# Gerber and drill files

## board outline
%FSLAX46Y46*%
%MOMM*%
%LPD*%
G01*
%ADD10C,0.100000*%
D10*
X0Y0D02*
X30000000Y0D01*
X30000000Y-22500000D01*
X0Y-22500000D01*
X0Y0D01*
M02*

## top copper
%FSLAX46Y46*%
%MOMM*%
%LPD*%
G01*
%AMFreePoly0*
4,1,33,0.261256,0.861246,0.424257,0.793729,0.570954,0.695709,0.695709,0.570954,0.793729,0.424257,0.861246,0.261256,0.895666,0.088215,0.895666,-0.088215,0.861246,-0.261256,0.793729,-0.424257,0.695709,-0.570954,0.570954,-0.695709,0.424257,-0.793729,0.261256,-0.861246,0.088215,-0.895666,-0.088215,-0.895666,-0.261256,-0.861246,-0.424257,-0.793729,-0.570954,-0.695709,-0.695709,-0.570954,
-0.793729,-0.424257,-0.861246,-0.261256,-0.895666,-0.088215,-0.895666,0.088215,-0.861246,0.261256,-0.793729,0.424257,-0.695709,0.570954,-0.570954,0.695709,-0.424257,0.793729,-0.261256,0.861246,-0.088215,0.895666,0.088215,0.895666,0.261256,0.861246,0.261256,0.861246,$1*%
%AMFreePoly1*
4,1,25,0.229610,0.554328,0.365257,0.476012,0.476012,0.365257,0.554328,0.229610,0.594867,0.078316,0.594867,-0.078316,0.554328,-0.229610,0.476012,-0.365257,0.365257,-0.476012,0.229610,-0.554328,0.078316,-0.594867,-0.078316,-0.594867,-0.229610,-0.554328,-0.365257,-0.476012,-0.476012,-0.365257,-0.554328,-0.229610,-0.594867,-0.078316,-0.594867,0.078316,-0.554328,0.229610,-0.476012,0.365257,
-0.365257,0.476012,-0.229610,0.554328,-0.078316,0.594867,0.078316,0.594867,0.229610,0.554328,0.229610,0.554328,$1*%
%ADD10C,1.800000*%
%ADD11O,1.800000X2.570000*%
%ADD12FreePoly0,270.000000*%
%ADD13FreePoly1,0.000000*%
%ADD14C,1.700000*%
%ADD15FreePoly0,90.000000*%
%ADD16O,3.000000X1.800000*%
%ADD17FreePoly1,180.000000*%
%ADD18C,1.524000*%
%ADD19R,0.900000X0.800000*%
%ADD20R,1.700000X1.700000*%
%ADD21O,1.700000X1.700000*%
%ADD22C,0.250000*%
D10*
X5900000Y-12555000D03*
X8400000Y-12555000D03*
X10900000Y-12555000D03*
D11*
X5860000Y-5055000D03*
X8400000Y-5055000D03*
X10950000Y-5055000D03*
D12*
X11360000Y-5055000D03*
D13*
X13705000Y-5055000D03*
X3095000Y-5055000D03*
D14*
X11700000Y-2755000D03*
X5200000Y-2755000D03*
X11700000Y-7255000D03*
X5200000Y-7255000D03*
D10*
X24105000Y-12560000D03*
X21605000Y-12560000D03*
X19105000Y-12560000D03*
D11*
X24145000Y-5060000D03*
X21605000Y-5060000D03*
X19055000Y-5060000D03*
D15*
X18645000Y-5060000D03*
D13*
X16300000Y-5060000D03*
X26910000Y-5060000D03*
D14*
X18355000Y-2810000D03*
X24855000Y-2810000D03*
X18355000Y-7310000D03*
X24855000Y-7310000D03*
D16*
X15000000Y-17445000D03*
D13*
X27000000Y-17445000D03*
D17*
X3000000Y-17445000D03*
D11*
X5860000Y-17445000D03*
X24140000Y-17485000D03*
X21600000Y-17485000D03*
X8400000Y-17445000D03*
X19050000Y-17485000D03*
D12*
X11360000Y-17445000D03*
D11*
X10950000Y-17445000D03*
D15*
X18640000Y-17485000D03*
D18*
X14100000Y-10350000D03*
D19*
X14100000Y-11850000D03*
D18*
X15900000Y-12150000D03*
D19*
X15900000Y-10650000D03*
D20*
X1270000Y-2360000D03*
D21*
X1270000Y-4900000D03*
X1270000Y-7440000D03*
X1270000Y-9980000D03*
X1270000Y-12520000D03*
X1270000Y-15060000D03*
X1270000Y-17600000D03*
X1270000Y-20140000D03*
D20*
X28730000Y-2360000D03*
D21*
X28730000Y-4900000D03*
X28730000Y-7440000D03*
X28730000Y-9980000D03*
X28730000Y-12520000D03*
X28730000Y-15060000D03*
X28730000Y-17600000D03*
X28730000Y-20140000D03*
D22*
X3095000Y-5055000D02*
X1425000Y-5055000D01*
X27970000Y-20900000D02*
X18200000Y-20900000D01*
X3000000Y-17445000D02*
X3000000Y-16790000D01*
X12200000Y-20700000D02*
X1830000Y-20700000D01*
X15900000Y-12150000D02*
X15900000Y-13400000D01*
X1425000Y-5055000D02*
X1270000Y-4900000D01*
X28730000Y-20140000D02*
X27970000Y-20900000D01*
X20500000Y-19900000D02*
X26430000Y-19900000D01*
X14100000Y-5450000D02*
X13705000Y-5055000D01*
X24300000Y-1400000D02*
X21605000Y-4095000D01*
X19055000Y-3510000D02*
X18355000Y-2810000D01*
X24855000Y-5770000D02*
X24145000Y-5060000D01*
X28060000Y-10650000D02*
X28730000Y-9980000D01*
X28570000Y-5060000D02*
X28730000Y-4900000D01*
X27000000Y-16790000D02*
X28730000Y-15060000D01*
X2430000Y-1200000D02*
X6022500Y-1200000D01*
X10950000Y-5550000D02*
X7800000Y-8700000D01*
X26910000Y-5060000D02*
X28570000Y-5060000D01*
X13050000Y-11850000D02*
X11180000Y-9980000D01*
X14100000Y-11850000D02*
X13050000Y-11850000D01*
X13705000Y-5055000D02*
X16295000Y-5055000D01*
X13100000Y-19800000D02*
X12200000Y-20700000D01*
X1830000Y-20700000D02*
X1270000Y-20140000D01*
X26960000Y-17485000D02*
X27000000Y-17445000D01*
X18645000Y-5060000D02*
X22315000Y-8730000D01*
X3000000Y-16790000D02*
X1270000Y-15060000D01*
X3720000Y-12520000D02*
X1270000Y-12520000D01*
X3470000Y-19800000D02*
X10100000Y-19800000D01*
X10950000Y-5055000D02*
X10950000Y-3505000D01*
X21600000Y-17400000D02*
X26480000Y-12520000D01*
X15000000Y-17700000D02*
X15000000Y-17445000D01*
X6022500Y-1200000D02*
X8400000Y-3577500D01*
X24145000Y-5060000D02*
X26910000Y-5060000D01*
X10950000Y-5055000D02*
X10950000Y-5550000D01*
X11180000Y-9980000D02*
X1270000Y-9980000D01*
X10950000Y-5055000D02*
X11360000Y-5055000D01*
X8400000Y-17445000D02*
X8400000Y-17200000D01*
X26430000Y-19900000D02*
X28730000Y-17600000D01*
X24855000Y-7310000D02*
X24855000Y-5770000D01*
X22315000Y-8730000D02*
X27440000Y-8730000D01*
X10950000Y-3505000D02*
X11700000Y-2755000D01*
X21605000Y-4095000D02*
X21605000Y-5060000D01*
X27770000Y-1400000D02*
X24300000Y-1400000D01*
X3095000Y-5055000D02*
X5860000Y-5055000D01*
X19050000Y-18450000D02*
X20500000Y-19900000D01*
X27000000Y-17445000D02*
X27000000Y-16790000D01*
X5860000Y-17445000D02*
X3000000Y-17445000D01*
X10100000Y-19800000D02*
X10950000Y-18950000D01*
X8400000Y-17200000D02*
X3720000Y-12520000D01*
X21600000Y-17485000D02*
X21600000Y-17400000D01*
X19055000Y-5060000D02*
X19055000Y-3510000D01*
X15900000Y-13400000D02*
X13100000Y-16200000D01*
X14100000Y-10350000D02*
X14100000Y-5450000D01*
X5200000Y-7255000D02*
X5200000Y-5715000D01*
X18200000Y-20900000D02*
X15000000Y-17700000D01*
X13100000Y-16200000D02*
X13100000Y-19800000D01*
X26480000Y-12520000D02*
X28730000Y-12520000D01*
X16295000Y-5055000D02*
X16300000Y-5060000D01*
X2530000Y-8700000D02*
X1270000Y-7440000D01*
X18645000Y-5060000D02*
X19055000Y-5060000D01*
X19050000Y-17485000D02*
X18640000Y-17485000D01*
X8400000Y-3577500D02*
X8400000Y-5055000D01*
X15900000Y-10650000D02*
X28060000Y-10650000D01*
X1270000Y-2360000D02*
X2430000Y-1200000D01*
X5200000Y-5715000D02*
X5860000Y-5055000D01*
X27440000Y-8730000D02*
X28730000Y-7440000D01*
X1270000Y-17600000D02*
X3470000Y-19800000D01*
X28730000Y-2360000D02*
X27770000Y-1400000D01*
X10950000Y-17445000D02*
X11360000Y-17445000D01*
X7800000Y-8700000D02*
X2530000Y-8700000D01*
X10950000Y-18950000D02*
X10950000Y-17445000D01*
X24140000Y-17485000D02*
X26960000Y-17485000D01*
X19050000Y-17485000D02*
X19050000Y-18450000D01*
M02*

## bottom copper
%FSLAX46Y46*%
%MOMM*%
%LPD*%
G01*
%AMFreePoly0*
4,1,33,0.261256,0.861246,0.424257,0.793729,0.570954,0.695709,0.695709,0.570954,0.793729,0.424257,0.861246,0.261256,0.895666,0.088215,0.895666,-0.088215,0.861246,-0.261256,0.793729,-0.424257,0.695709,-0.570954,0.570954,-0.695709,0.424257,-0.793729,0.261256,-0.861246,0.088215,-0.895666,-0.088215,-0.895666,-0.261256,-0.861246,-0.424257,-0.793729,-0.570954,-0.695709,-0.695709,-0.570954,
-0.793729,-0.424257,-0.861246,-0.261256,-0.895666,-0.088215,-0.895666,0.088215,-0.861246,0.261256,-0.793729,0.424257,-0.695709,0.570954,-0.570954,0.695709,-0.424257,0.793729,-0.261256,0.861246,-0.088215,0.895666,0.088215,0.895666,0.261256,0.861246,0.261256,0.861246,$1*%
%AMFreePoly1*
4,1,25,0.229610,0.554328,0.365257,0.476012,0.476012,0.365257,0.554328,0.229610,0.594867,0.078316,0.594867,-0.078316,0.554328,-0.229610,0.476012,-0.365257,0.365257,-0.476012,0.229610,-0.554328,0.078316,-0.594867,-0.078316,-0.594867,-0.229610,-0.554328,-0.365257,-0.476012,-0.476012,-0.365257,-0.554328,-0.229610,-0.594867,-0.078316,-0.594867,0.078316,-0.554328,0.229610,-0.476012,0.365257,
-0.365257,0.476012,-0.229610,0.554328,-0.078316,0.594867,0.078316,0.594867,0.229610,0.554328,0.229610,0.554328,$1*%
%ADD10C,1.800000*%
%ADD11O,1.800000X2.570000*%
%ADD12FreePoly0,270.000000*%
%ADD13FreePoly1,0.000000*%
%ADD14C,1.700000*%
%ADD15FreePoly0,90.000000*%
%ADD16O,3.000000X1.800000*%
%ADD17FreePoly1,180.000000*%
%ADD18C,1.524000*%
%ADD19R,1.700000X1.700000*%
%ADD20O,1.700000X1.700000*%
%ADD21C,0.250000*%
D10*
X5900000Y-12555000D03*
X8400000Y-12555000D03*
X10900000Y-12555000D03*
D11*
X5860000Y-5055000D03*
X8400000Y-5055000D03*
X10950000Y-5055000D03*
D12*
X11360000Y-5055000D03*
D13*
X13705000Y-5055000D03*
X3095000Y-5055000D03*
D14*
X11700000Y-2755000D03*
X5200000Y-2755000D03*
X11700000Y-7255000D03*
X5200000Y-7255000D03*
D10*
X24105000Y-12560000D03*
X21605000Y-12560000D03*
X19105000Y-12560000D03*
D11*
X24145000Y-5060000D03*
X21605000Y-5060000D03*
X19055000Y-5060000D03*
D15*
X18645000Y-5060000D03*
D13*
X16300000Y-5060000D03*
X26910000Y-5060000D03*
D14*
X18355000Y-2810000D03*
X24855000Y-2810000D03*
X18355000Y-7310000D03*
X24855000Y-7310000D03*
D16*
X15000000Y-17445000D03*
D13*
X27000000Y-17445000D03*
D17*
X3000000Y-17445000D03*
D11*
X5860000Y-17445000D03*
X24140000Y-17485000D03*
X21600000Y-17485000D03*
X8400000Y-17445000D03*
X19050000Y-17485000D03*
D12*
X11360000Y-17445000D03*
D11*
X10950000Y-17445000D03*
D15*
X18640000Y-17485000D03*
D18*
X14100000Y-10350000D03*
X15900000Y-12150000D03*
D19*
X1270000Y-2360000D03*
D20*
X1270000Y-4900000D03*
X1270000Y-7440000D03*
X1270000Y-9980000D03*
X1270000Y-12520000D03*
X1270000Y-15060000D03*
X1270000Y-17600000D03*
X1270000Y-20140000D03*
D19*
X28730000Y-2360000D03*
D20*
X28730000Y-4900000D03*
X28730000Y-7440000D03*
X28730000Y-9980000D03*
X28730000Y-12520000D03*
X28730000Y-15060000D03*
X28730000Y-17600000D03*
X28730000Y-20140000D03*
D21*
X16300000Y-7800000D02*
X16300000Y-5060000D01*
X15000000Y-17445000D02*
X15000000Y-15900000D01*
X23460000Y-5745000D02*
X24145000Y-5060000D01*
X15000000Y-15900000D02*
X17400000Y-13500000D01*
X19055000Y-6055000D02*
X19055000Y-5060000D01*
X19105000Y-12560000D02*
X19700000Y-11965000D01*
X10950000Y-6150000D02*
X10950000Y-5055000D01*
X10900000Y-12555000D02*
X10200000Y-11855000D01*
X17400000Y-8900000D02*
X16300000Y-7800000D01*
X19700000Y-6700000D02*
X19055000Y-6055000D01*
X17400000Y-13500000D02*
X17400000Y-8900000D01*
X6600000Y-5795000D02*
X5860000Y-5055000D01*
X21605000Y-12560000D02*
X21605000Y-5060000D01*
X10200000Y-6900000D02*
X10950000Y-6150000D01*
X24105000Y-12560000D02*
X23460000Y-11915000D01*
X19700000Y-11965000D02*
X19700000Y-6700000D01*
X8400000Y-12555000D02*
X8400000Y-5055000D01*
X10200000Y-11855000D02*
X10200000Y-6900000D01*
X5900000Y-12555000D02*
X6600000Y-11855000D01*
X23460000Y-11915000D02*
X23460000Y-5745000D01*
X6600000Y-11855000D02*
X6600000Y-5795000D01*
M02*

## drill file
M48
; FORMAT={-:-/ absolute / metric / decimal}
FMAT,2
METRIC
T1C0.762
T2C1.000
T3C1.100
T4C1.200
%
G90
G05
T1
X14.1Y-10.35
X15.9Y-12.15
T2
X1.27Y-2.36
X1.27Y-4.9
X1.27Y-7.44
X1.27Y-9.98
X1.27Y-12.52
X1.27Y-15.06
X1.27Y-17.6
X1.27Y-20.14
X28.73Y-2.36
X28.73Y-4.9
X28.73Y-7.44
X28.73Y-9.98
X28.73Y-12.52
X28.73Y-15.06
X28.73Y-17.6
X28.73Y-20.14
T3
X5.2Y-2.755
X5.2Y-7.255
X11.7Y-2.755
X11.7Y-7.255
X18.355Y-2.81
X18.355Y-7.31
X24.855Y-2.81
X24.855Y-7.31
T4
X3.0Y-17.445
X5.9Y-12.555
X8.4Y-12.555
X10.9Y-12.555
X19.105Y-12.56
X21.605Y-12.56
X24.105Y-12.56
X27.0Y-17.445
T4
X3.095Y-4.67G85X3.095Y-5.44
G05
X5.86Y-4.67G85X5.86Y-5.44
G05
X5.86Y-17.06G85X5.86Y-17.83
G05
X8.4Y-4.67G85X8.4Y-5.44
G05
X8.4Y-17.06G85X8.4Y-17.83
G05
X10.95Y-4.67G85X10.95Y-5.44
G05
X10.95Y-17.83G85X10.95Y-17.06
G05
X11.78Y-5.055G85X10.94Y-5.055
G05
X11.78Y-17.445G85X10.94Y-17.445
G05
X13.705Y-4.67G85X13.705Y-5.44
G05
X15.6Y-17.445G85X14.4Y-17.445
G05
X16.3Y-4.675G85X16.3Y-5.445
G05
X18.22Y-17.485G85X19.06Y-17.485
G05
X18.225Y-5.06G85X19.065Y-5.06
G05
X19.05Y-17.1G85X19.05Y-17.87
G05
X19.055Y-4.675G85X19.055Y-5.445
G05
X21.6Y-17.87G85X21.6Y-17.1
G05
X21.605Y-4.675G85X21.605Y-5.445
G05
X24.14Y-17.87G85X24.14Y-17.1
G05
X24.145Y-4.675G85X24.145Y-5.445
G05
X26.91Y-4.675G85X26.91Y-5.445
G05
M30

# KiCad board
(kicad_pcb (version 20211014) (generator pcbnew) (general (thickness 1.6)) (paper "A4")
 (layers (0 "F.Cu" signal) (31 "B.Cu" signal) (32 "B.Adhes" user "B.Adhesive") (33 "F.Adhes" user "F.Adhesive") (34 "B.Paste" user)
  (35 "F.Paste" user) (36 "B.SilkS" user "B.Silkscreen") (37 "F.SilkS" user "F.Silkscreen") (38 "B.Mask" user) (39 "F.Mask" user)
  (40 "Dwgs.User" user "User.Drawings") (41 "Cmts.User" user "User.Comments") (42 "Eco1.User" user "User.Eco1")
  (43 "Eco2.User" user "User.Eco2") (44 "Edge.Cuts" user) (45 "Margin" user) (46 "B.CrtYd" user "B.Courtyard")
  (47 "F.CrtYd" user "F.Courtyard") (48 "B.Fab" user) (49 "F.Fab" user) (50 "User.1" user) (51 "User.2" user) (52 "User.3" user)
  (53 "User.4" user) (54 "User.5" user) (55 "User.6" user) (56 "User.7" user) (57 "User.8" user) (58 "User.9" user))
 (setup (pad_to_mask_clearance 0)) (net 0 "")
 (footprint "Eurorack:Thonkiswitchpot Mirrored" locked (layer "F.Cu") (at 8.4 5.055)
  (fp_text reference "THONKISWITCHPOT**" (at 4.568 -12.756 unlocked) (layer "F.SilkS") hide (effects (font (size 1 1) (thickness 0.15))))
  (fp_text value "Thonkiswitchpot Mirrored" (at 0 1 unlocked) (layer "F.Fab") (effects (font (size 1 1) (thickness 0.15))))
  (pad "1" thru_hole circle locked (at -2.5 7.5 270) (size 1.8 1.8) (drill 1.2) (layers *.Cu *.Mask))
  (pad "2" thru_hole circle locked (at 0 7.5 270) (size 1.8 1.8) (drill 1.2) (layers *.Cu *.Mask))
  (pad "3" thru_hole circle locked (at 2.5 7.5 270) (size 1.8 1.8) (drill 1.2) (layers *.Cu *.Mask))
  (pad "4" thru_hole oval locked (at -2.54 0) (size 1.8 2.57) (drill oval 1.2 1.97) (layers *.Cu *.Mask))
  (pad "5" thru_hole oval locked (at 0 0) (size 1.8 2.57) (drill oval 1.2 1.97) (layers *.Cu *.Mask))
  (pad "6" thru_hole oval locked (at 2.55 0) (size 1.8 2.57) (drill oval 1.2 1.97) (layers *.Cu *.Mask))
  (pad "6" thru_hole custom locked (at 2.96 0 270) (size 1.8 1.8) (drill oval 1.2 2.04) (layers *.Cu *.Mask)
   (options (clearance outline) (anchor circle)) (primitives))
  (pad "7" thru_hole custom locked (at 5.305 0) (size 1.2 1.2) (drill oval 1.2 1.97) (layers *.Cu *.Mask)
   (options (clearance outline) (anchor circle)) (primitives))
  (pad "8" thru_hole custom locked (at -5.305 0) (size 1.2 1.97) (drill oval 1.2 1.97) (layers *.Cu *.Mask)
   (options (clearance outline) (anchor circle)) (primitives))
  (pad "9" thru_hole circle locked (at 3.3 -2.3 270) (size 1.7 1.7) (drill 1.1) (layers *.Cu *.Mask))
  (pad "10" thru_hole circle locked (at -3.2 -2.3 270) (size 1.7 1.7) (drill 1.1) (layers *.Cu *.Mask))
  (pad "11" thru_hole circle locked (at 3.3 2.2 270) (size 1.7 1.7) (drill 1.1) (layers *.Cu *.Mask))
  (pad "12" thru_hole circle locked (at -3.2 2.2 270) (size 1.7 1.7) (drill 1.1) (layers *.Cu *.Mask)))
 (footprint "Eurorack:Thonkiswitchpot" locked (layer "F.Cu") (at 21.605 5.06)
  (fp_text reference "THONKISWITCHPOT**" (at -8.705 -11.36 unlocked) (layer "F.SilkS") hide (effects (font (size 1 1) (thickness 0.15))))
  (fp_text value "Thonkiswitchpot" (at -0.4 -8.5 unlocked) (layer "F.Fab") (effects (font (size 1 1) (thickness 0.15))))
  (pad "1" thru_hole circle locked (at 2.5 7.5 90) (size 1.8 1.8) (drill 1.2) (layers *.Cu *.Mask))
  (pad "2" thru_hole circle locked (at 0 7.5 90) (size 1.8 1.8) (drill 1.2) (layers *.Cu *.Mask))
  (pad "3" thru_hole circle locked (at -2.5 7.5 90) (size 1.8 1.8) (drill 1.2) (layers *.Cu *.Mask))
  (pad "4" thru_hole oval locked (at 2.54 0) (size 1.8 2.57) (drill oval 1.2 1.97) (layers *.Cu *.Mask))
  (pad "5" thru_hole oval locked (at 0 0) (size 1.8 2.57) (drill oval 1.2 1.97) (layers *.Cu *.Mask))
  (pad "6" thru_hole oval locked (at -2.55 0) (size 1.8 2.57) (drill oval 1.2 1.97) (layers *.Cu *.Mask))
  (pad "6" thru_hole custom locked (at -2.96 0 90) (size 1.8 1.8) (drill oval 1.2 2.04) (layers *.Cu *.Mask)
   (options (clearance outline) (anchor circle)) (primitives))
  (pad "7" thru_hole custom locked (at -5.305 0) (size 1.2 1.2) (drill oval 1.2 1.97) (layers *.Cu *.Mask)
   (options (clearance outline) (anchor circle)) (primitives))
  (pad "8" thru_hole custom locked (at 5.305 0) (size 1.2 1.97) (drill oval 1.2 1.97) (layers *.Cu *.Mask)
   (options (clearance outline) (anchor circle)) (primitives))
  (pad "9" thru_hole circle locked (at -3.25 -2.25 90) (size 1.7 1.7) (drill 1.1) (layers *.Cu *.Mask))
  (pad "10" thru_hole circle locked (at 3.25 -2.25 90) (size 1.7 1.7) (drill 1.1) (layers *.Cu *.Mask))
  (pad "11" thru_hole circle locked (at -3.25 2.25 90) (size 1.7 1.7) (drill 1.1) (layers *.Cu *.Mask))
  (pad "12" thru_hole circle locked (at 3.25 2.25 90) (size 1.7 1.7) (drill 1.1) (layers *.Cu *.Mask)))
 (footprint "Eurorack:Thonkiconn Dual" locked (layer "F.Cu") (at 15 17.445)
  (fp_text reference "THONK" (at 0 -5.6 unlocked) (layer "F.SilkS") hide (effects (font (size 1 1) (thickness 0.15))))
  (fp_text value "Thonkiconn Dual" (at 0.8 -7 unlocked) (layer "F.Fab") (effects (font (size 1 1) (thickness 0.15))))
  (pad "1" thru_hole oval locked (at 0 0 180) (size 3 1.8) (drill oval 2.4 1.2) (layers *.Cu *.Mask))
  (pad "3" thru_hole custom locked (at 12 0) (size 1.2 1.2) (drill 1.2) (layers *.Cu *.Mask) (options (clearance outline) (anchor circle))
   (primitives))
  (pad "3" thru_hole custom locked (at -12 0 180) (size 1.2 1.2) (drill 1.2) (layers *.Cu *.Mask)
   (options (clearance outline) (anchor circle)) (primitives))
  (pad "4" thru_hole oval locked (at -9.14 0) (size 1.8 2.57) (drill oval 1.2 1.97) (layers *.Cu *.Mask))
  (pad "4" thru_hole oval locked (at 9.14 0.04 180) (size 1.8 2.57) (drill oval 1.2 1.97) (layers *.Cu *.Mask))
  (pad "5" thru_hole oval locked (at 6.6 0.04 180) (size 1.8 2.57) (drill oval 1.2 1.97) (layers *.Cu *.Mask))
  (pad "5" thru_hole oval locked (at -6.6 0) (size 1.8 2.57) (drill oval 1.2 1.97) (layers *.Cu *.Mask))
  (pad "6" thru_hole oval locked (at 4.05 0.04) (size 1.8 2.57) (drill oval 1.2 1.97) (layers *.Cu *.Mask))
  (pad "6" thru_hole custom locked (at -3.64 0 270) (size 1.8 1.8) (drill oval 1.2 2.04) (layers *.Cu *.Mask)
   (options (clearance outline) (anchor circle)) (primitives))
  (pad "6" thru_hole oval locked (at -4.05 0 180) (size 1.8 2.57) (drill oval 1.2 1.97) (layers *.Cu *.Mask))
  (pad "6" thru_hole custom locked (at 3.64 0.04 90) (size 1.8 1.8) (drill oval 1.2 2.04) (layers *.Cu *.Mask)
   (options (clearance outline) (anchor circle)) (primitives)))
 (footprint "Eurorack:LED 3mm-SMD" (layer "F.Cu") (at 15 11.25)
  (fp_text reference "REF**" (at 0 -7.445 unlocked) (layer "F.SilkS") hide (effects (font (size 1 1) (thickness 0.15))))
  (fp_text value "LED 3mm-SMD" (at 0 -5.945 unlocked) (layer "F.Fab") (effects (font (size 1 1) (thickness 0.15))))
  (pad "1" thru_hole circle (at -0.9 -0.9) (size 1.524 1.524) (drill 0.762) (layers *.Cu *.Mask))
  (pad "2" smd rect (at -0.9 0.6) (size 0.9 0.8) (layers "F.Cu" "F.Paste" "F.Mask"))
  (pad "3" thru_hole circle (at 0.9 0.9) (size 1.524 1.524) (drill 0.762) (layers *.Cu *.Mask))
  (pad "4" smd rect (at 0.9 -0.6) (size 0.9 0.8) (layers "F.Cu" "F.Paste" "F.Mask")))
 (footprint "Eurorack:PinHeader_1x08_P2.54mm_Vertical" (layer "B.Cu") (at 1.27 2.36 180)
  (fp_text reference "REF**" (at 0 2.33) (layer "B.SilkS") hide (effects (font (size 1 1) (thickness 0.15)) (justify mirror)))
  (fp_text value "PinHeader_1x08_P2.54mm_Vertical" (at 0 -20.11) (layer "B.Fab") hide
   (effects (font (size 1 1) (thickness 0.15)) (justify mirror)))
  (pad "1" thru_hole rect (at 0 0 180) (size 1.7 1.7) (drill 1) (layers *.Cu *.Mask))
  (pad "2" thru_hole oval (at 0 -2.54 180) (size 1.7 1.7) (drill 1) (layers *.Cu *.Mask))
  (pad "3" thru_hole oval (at 0 -5.08 180) (size 1.7 1.7) (drill 1) (layers *.Cu *.Mask))
  (pad "4" thru_hole oval (at 0 -7.62 180) (size 1.7 1.7) (drill 1) (layers *.Cu *.Mask))
  (pad "5" thru_hole oval (at 0 -10.16 180) (size 1.7 1.7) (drill 1) (layers *.Cu *.Mask))
  (pad "6" thru_hole oval (at 0 -12.7 180) (size 1.7 1.7) (drill 1) (layers *.Cu *.Mask))
  (pad "7" thru_hole oval (at 0 -15.24 180) (size 1.7 1.7) (drill 1) (layers *.Cu *.Mask))
  (pad "8" thru_hole oval (at 0 -17.78 180) (size 1.7 1.7) (drill 1) (layers *.Cu *.Mask)))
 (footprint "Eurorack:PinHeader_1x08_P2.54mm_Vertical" (layer "B.Cu") (at 28.73 2.36 180)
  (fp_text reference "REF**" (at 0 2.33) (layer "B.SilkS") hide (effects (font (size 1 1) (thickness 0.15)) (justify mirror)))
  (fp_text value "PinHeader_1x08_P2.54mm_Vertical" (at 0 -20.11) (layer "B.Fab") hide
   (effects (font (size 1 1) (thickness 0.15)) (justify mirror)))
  (pad "1" thru_hole rect (at 0 0 180) (size 1.7 1.7) (drill 1) (layers *.Cu *.Mask))
  (pad "2" thru_hole oval (at 0 -2.54 180) (size 1.7 1.7) (drill 1) (layers *.Cu *.Mask))
  (pad "3" thru_hole oval (at 0 -5.08 180) (size 1.7 1.7) (drill 1) (layers *.Cu *.Mask))
  (pad "4" thru_hole oval (at 0 -7.62 180) (size 1.7 1.7) (drill 1) (layers *.Cu *.Mask))
  (pad "5" thru_hole oval (at 0 -10.16 180) (size 1.7 1.7) (drill 1) (layers *.Cu *.Mask))
  (pad "6" thru_hole oval (at 0 -12.7 180) (size 1.7 1.7) (drill 1) (layers *.Cu *.Mask))
  (pad "7" thru_hole oval (at 0 -15.24 180) (size 1.7 1.7) (drill 1) (layers *.Cu *.Mask))
  (pad "8" thru_hole oval (at 0 -17.78 180) (size 1.7 1.7) (drill 1) (layers *.Cu *.Mask)))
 (gr_rect (start 0 0) (end 30 22.5) (layer "Edge.Cuts") (width 0.1) (fill none))
 (segment (start 3.095 5.055) (end 1.425 5.055) (width 0.25) (layer "F.Cu") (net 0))
 (segment (start 27.97 20.9) (end 18.2 20.9) (width 0.25) (layer "F.Cu") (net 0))
 (segment (start 3 17.445) (end 3 16.79) (width 0.25) (layer "F.Cu") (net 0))
 (segment (start 12.2 20.7) (end 1.83 20.7) (width 0.25) (layer "F.Cu") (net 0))
 (segment (start 15.9 12.15) (end 15.9 13.4) (width 0.25) (layer "F.Cu") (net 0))
 (segment (start 1.425 5.055) (end 1.27 4.9) (width 0.25) (layer "F.Cu") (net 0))
 (segment (start 28.73 20.14) (end 27.97 20.9) (width 0.25) (layer "F.Cu") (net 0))
 (segment (start 20.5 19.9) (end 26.43 19.9) (width 0.25) (layer "F.Cu") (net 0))
 (segment (start 14.1 5.45) (end 13.705 5.055) (width 0.25) (layer "F.Cu") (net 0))
 (segment (start 24.3 1.4) (end 21.605 4.095) (width 0.25) (layer "F.Cu") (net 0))
 (segment (start 19.055 3.51) (end 18.355 2.81) (width 0.25) (layer "F.Cu") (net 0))
 (segment (start 24.855 5.77) (end 24.145 5.06) (width 0.25) (layer "F.Cu") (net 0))
 (segment (start 28.06 10.65) (end 28.73 9.98) (width 0.25) (layer "F.Cu") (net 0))
 (segment (start 28.57 5.06) (end 28.73 4.9) (width 0.25) (layer "F.Cu") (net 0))
 (segment (start 27 16.79) (end 28.73 15.06) (width 0.25) (layer "F.Cu") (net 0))
 (segment (start 2.43 1.2) (end 6.0225 1.2) (width 0.25) (layer "F.Cu") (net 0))
 (segment (start 10.95 5.55) (end 7.8 8.7) (width 0.25) (layer "F.Cu") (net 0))
 (segment (start 26.91 5.06) (end 28.57 5.06) (width 0.25) (layer "F.Cu") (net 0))
 (segment (start 13.05 11.85) (end 11.18 9.98) (width 0.25) (layer "F.Cu") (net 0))
 (segment (start 14.1 11.85) (end 13.05 11.85) (width 0.25) (layer "F.Cu") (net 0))
 (segment (start 13.705 5.055) (end 16.295 5.055) (width 0.25) (layer "F.Cu") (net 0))
 (segment (start 13.1 19.8) (end 12.2 20.7) (width 0.25) (layer "F.Cu") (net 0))
 (segment (start 1.83 20.7) (end 1.27 20.14) (width 0.25) (layer "F.Cu") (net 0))
 (segment (start 26.96 17.485) (end 27 17.445) (width 0.25) (layer "F.Cu") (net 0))
 (segment (start 18.645 5.06) (end 22.315 8.73) (width 0.25) (layer "F.Cu") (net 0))
 (segment (start 3 16.79) (end 1.27 15.06) (width 0.25) (layer "F.Cu") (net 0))
 (segment (start 3.72 12.52) (end 1.27 12.52) (width 0.25) (layer "F.Cu") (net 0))
 (segment (start 3.47 19.8) (end 10.1 19.8) (width 0.25) (layer "F.Cu") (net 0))
 (segment (start 10.95 5.055) (end 10.95 3.505) (width 0.25) (layer "F.Cu") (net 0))
 (segment (start 21.6 17.4) (end 26.48 12.52) (width 0.25) (layer "F.Cu") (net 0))
 (segment (start 15 17.7) (end 15 17.445) (width 0.25) (layer "F.Cu") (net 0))
 (segment (start 6.0225 1.2) (end 8.4 3.5775) (width 0.25) (layer "F.Cu") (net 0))
 (segment (start 24.145 5.06) (end 26.91 5.06) (width 0.25) (layer "F.Cu") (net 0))
 (segment (start 10.95 5.055) (end 10.95 5.55) (width 0.25) (layer "F.Cu") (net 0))
 (segment (start 11.18 9.98) (end 1.27 9.98) (width 0.25) (layer "F.Cu") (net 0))
 (segment (start 10.95 5.055) (end 11.36 5.055) (width 0.25) (layer "F.Cu") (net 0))
 (segment (start 8.4 17.445) (end 8.4 17.2) (width 0.25) (layer "F.Cu") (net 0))
 (segment (start 26.43 19.9) (end 28.73 17.6) (width 0.25) (layer "F.Cu") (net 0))
 (segment (start 24.855 7.31) (end 24.855 5.77) (width 0.25) (layer "F.Cu") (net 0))
 (segment (start 22.315 8.73) (end 27.44 8.73) (width 0.25) (layer "F.Cu") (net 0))
 (segment (start 10.95 3.505) (end 11.7 2.755) (width 0.25) (layer "F.Cu") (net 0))
 (segment (start 21.605 4.095) (end 21.605 5.06) (width 0.25) (layer "F.Cu") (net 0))
 (segment (start 27.77 1.4) (end 24.3 1.4) (width 0.25) (layer "F.Cu") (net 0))
 (segment (start 3.095 5.055) (end 5.86 5.055) (width 0.25) (layer "F.Cu") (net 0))
 (segment (start 19.05 18.45) (end 20.5 19.9) (width 0.25) (layer "F.Cu") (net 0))
 (segment (start 27 17.445) (end 27 16.79) (width 0.25) (layer "F.Cu") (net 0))
 (segment (start 5.86 17.445) (end 3 17.445) (width 0.25) (layer "F.Cu") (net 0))
 (segment (start 10.1 19.8) (end 10.95 18.95) (width 0.25) (layer "F.Cu") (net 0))
 (segment (start 8.4 17.2) (end 3.72 12.52) (width 0.25) (layer "F.Cu") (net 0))
 (segment (start 21.6 17.485) (end 21.6 17.4) (width 0.25) (layer "F.Cu") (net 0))
 (segment (start 19.055 5.06) (end 19.055 3.51) (width 0.25) (layer "F.Cu") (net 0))
 (segment (start 15.9 13.4) (end 13.1 16.2) (width 0.25) (layer "F.Cu") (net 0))
 (segment (start 14.1 10.35) (end 14.1 5.45) (width 0.25) (layer "F.Cu") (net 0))
 (segment (start 5.2 7.255) (end 5.2 5.715) (width 0.25) (layer "F.Cu") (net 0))
 (segment (start 18.2 20.9) (end 15 17.7) (width 0.25) (layer "F.Cu") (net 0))
 (segment (start 13.1 16.2) (end 13.1 19.8) (width 0.25) (layer "F.Cu") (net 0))
 (segment (start 26.48 12.52) (end 28.73 12.52) (width 0.25) (layer "F.Cu") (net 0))
 (segment (start 16.295 5.055) (end 16.3 5.06) (width 0.25) (layer "F.Cu") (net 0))
 (segment (start 2.53 8.7) (end 1.27 7.44) (width 0.25) (layer "F.Cu") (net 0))
 (segment (start 18.645 5.06) (end 19.055 5.06) (width 0.25) (layer "F.Cu") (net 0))
 (segment (start 19.05 17.485) (end 18.64 17.485) (width 0.25) (layer "F.Cu") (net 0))
 (segment (start 8.4 3.5775) (end 8.4 5.055) (width 0.25) (layer "F.Cu") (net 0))
 (segment (start 15.9 10.65) (end 28.06 10.65) (width 0.25) (layer "F.Cu") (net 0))
 (segment (start 1.27 2.36) (end 2.43 1.2) (width 0.25) (layer "F.Cu") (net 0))
 (segment (start 5.2 5.715) (end 5.86 5.055) (width 0.25) (layer "F.Cu") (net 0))
 (segment (start 27.44 8.73) (end 28.73 7.44) (width 0.25) (layer "F.Cu") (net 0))
 (segment (start 1.27 17.6) (end 3.47 19.8) (width 0.25) (layer "F.Cu") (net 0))
 (segment (start 28.73 2.36) (end 27.77 1.4) (width 0.25) (layer "F.Cu") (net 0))
 (segment (start 10.95 17.445) (end 11.36 17.445) (width 0.25) (layer "F.Cu") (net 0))
 (segment (start 7.8 8.7) (end 2.53 8.7) (width 0.25) (layer "F.Cu") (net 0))
 (segment (start 10.95 18.95) (end 10.95 17.445) (width 0.25) (layer "F.Cu") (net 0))
 (segment (start 24.14 17.485) (end 26.96 17.485) (width 0.25) (layer "F.Cu") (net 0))
 (segment (start 19.05 17.485) (end 19.05 18.45) (width 0.25) (layer "F.Cu") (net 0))
 (segment (start 16.3 7.8) (end 16.3 5.06) (width 0.25) (layer "B.Cu") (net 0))
 (segment (start 15 17.445) (end 15 15.9) (width 0.25) (layer "B.Cu") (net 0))
 (segment (start 23.46 5.745) (end 24.145 5.06) (width 0.25) (layer "B.Cu") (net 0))
 (segment (start 15 15.9) (end 17.4 13.5) (width 0.25) (layer "B.Cu") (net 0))
 (segment (start 19.055 6.055) (end 19.055 5.06) (width 0.25) (layer "B.Cu") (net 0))
 (segment (start 19.105 12.56) (end 19.7 11.965) (width 0.25) (layer "B.Cu") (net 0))
 (segment (start 10.95 6.15) (end 10.95 5.055) (width 0.25) (layer "B.Cu") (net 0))
 (segment (start 10.9 12.555) (end 10.2 11.855) (width 0.25) (layer "B.Cu") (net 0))
 (segment (start 17.4 8.9) (end 16.3 7.8) (width 0.25) (layer "B.Cu") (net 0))
 (segment (start 19.7 6.7) (end 19.055 6.055) (width 0.25) (layer "B.Cu") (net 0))
 (segment (start 17.4 13.5) (end 17.4 8.9) (width 0.25) (layer "B.Cu") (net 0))
 (segment (start 6.6 5.795) (end 5.86 5.055) (width 0.25) (layer "B.Cu") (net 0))
 (segment (start 21.605 12.56) (end 21.605 5.06) (width 0.25) (layer "B.Cu") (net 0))
 (segment (start 10.2 6.9) (end 10.95 6.15) (width 0.25) (layer "B.Cu") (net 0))
 (segment (start 24.105 12.56) (end 23.46 11.915) (width 0.25) (layer "B.Cu") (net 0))
 (segment (start 19.7 11.965) (end 19.7 6.7) (width 0.25) (layer "B.Cu") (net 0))
 (segment (start 8.4 12.555) (end 8.4 5.055) (width 0.25) (layer "B.Cu") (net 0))
 (segment (start 10.2 11.855) (end 10.2 6.9) (width 0.25) (layer "B.Cu") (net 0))
 (segment (start 5.9 12.555) (end 6.6 11.855) (width 0.25) (layer "B.Cu") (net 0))
 (segment (start 23.46 11.915) (end 23.46 5.745) (width 0.25) (layer "B.Cu") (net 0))
 (segment (start 6.6 11.855) (end 6.6 5.795) (width 0.25) (layer "B.Cu") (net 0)))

